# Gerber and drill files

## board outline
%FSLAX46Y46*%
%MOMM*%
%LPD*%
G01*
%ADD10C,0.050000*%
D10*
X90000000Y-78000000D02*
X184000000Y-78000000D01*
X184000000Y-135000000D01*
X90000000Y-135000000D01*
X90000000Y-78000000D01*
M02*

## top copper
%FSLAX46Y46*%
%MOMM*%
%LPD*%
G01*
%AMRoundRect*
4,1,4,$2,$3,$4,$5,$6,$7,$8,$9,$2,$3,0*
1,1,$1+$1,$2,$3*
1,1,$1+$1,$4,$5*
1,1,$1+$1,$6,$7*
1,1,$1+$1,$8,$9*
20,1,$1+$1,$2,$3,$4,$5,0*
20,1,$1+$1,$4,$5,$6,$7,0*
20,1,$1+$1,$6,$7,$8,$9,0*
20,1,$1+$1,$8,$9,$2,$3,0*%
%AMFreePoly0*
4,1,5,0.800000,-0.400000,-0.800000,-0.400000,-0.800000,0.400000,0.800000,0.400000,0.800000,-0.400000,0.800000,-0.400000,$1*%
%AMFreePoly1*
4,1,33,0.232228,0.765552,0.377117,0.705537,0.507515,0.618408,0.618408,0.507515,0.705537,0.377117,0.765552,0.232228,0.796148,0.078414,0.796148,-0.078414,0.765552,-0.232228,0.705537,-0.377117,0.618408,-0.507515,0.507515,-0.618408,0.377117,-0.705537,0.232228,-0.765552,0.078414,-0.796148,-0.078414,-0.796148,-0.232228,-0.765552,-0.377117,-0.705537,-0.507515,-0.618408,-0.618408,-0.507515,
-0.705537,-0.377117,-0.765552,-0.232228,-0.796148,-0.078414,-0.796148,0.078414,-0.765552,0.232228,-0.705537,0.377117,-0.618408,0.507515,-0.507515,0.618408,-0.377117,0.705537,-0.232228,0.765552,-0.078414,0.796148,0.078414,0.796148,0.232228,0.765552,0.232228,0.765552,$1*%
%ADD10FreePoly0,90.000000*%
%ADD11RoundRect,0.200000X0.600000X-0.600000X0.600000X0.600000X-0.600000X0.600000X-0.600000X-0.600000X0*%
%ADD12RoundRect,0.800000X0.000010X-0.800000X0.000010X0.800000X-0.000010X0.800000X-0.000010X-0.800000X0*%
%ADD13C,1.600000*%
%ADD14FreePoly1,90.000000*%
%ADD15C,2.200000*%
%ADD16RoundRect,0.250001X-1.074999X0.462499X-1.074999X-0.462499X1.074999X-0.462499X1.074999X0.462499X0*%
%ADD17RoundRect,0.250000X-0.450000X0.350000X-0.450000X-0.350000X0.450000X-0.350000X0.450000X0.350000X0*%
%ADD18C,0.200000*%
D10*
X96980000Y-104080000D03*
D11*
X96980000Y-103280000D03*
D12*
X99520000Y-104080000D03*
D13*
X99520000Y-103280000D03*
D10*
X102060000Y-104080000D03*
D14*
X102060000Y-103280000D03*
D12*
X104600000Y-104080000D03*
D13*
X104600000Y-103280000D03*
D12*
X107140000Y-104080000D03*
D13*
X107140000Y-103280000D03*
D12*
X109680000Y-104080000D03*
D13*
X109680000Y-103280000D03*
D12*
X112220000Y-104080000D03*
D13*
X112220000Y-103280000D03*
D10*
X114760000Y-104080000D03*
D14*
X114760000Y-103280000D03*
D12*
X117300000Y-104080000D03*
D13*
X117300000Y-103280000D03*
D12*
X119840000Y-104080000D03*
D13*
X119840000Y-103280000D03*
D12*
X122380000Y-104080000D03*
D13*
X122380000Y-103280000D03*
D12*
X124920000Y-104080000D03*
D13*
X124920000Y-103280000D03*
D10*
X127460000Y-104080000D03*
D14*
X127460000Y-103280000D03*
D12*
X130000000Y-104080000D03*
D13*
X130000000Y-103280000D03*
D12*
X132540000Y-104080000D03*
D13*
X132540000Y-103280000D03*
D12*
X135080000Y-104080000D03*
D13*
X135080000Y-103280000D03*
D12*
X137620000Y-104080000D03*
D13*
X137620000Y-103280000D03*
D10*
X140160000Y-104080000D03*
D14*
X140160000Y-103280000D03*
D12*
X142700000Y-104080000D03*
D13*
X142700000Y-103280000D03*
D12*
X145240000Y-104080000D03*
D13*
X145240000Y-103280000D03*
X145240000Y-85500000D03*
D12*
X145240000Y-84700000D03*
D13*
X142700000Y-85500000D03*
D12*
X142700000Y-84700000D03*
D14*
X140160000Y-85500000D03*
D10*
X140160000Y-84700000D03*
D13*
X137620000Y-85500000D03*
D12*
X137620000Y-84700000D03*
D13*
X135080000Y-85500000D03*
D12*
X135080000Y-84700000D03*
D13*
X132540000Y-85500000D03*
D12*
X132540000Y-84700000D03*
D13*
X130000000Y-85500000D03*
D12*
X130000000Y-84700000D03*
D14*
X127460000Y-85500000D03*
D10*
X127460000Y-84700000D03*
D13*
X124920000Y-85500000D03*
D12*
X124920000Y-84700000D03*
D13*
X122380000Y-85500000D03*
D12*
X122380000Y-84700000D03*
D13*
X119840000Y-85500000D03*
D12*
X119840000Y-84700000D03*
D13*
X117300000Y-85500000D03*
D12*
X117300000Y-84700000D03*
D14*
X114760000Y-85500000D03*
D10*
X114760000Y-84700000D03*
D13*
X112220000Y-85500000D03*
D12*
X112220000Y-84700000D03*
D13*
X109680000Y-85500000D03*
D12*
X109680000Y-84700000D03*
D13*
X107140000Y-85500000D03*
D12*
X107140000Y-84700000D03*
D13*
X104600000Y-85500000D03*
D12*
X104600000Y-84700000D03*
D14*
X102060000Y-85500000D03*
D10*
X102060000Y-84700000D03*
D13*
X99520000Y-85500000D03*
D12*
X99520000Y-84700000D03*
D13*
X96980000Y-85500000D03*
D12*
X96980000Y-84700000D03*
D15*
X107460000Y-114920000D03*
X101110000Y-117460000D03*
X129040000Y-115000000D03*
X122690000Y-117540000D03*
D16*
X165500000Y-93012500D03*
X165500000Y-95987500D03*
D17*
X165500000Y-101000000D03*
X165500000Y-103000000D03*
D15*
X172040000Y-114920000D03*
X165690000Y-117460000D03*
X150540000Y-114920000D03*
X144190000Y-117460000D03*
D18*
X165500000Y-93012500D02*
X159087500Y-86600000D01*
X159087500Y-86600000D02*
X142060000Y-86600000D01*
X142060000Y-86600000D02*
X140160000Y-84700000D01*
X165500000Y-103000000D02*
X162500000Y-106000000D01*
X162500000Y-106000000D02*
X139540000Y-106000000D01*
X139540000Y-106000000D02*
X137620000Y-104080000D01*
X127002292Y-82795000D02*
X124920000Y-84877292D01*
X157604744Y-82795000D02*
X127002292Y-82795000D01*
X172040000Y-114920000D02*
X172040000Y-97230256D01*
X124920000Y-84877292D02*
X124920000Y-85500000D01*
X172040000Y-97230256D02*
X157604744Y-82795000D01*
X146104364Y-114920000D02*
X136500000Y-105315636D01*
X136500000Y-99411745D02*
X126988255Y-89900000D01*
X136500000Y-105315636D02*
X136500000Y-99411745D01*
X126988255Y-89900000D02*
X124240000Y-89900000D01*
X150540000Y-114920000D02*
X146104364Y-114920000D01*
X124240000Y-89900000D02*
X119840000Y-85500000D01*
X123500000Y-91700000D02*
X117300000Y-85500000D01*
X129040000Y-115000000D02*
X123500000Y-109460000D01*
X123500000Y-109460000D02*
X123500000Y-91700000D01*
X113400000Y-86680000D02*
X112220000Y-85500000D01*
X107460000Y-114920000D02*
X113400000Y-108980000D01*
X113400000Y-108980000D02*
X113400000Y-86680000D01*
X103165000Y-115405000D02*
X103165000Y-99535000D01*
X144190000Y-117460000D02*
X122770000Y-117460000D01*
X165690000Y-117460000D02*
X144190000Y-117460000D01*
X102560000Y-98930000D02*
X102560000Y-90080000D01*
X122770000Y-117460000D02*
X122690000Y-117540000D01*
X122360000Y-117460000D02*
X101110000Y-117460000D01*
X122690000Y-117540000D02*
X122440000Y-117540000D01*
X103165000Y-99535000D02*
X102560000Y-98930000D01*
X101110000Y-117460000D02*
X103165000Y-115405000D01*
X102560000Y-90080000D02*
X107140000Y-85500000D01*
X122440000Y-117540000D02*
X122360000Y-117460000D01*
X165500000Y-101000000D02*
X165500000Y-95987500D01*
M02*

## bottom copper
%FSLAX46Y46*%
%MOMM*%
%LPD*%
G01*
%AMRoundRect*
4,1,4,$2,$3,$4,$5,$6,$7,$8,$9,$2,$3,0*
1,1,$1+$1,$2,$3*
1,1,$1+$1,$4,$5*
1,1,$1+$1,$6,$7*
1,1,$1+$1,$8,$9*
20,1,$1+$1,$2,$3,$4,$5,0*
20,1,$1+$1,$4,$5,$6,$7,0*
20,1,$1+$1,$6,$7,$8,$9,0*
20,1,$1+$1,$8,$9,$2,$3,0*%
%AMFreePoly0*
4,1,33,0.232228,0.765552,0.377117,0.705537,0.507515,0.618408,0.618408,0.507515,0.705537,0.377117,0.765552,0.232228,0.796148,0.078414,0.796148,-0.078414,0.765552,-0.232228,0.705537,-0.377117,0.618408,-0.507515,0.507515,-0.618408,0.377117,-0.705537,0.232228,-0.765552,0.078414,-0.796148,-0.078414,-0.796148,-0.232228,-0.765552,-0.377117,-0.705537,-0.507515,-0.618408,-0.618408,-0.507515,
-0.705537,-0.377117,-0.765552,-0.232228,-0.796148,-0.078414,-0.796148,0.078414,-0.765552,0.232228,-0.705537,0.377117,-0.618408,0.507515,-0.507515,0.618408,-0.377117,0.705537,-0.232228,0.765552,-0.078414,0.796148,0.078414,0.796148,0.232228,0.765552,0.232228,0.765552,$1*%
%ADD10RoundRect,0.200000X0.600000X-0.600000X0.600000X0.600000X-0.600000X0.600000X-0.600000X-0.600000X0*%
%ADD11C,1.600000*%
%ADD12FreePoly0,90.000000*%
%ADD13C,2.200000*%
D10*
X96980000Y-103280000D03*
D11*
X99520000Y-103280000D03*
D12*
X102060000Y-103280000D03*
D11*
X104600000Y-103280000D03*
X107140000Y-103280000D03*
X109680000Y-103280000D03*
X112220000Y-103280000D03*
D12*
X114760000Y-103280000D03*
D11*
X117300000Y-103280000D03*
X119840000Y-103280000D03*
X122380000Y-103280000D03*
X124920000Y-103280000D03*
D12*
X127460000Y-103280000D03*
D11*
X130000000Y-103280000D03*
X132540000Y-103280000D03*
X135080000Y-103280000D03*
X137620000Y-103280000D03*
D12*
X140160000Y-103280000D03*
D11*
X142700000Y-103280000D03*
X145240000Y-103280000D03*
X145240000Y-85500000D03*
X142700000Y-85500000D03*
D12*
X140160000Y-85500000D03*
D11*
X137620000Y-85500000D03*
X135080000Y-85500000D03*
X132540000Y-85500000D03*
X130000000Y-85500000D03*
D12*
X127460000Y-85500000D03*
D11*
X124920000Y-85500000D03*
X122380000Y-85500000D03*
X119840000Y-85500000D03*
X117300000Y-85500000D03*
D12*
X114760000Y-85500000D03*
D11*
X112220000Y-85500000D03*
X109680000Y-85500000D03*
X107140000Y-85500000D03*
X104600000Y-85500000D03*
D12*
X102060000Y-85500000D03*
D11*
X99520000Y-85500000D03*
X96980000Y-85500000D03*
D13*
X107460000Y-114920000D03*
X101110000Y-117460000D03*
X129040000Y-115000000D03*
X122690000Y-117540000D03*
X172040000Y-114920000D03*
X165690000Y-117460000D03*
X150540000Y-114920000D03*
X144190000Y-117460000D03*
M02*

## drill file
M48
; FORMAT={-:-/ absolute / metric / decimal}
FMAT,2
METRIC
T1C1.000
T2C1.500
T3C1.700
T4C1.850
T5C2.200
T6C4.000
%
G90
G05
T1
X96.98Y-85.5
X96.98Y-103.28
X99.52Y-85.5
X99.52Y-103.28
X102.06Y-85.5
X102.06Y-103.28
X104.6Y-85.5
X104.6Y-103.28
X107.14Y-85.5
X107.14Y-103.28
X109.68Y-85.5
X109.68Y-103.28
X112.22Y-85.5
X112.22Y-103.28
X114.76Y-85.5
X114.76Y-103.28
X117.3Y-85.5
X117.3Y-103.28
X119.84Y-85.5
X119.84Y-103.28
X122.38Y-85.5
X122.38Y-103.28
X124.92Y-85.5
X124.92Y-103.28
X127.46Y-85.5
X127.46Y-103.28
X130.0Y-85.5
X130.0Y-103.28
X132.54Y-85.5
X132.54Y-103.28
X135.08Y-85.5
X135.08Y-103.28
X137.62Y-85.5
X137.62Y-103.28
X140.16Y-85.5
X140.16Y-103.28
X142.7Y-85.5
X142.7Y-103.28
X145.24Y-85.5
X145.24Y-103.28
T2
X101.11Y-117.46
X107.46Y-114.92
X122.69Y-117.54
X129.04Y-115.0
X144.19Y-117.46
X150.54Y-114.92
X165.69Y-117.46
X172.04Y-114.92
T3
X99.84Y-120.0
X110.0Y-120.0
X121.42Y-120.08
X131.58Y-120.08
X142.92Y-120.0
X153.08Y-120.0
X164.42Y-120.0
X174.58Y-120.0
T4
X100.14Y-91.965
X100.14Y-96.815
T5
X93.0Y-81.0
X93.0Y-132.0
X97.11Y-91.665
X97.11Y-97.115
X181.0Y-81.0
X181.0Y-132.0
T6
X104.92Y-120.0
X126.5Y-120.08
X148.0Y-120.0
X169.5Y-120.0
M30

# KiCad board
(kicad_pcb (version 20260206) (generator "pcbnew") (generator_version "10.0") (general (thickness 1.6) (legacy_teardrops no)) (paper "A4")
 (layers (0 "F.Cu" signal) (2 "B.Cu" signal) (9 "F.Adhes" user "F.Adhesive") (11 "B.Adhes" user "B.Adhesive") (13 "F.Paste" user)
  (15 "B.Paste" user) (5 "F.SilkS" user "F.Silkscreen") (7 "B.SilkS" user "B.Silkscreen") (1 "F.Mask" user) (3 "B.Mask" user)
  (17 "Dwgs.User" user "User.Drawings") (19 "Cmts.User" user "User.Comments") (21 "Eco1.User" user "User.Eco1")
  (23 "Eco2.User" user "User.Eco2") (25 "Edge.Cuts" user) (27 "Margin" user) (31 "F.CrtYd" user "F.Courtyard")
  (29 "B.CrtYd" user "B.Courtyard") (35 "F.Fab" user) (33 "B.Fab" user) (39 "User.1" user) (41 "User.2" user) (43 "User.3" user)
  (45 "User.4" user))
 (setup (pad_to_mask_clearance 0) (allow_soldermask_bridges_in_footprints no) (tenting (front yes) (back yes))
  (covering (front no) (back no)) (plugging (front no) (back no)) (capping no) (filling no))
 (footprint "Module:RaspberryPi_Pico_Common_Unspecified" (layer "F.Cu") (at 121.11 94.39 90)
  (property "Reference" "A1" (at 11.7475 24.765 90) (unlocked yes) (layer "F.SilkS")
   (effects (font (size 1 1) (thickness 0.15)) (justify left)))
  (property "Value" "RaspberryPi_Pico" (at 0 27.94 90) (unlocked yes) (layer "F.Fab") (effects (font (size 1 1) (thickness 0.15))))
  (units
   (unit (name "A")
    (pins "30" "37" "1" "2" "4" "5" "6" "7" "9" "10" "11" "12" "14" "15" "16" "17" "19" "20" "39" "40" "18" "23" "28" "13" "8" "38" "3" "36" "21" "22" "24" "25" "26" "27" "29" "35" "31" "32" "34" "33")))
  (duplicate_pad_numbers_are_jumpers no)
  (pad "" np_thru_hole circle (at -2.725 -24 90) (size 2.2 2.2) (drill 2.2) (layers "*.Mask"))
  (pad "" np_thru_hole circle (at -2.425 -20.97 90) (size 1.85 1.85) (drill 1.85) (layers "*.Mask"))
  (pad "" np_thru_hole circle (at 2.425 -20.97 90) (size 1.85 1.85) (drill 1.85) (layers "*.Mask"))
  (pad "" np_thru_hole circle (at 2.725 -24 90) (size 2.2 2.2) (drill 2.2) (layers "*.Mask"))
  (pad "1" smd custom (at -9.69 -24.13 90) (size 1.6 0.8) (layers "F.Cu" "F.Mask") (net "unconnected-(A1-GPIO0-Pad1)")
   (options (clearance outline) (anchor rect)) (primitives))
  (pad "1" thru_hole roundrect (at -8.89 -24.13 90) (size 1.6 1.6) (drill 1) (layers "*.Cu" "*.Mask") (remove_unused_layers no)
   (roundrect_rratio 0.125) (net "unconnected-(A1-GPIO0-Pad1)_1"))
  (pad "2" smd roundrect (at -9.69 -21.59 90) (size 3.2 1.6) (layers "F.Cu" "F.Mask") (roundrect_rratio 0.5)
   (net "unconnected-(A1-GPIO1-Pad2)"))
  (pad "2" thru_hole circle (at -8.89 -21.59 90) (size 1.6 1.6) (drill 1) (layers "*.Cu" "*.Mask") (remove_unused_layers no)
   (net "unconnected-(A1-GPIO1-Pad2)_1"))
  (pad "3" smd custom (at -9.69 -19.05 90) (size 1.6 0.8) (layers "F.Cu" "F.Mask") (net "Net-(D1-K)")
   (options (clearance outline) (anchor rect)) (primitives))
  (pad "3" thru_hole custom (at -8.89 -19.05 90) (size 1.6 1.6) (drill 1) (layers "*.Cu" "*.Mask") (remove_unused_layers no)
   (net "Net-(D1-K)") (options (clearance outline) (anchor circle)) (primitives))
  (pad "4" smd roundrect (at -9.69 -16.51 90) (size 3.2 1.6) (layers "F.Cu" "F.Mask") (roundrect_rratio 0.5)
   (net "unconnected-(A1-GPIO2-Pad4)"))
  (pad "4" thru_hole circle (at -8.89 -16.51 90) (size 1.6 1.6) (drill 1) (layers "*.Cu" "*.Mask") (remove_unused_layers no)
   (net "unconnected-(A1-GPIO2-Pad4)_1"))
  (pad "5" smd roundrect (at -9.69 -13.97 90) (size 3.2 1.6) (layers "F.Cu" "F.Mask") (roundrect_rratio 0.5)
   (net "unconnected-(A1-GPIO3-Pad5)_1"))
  (pad "5" thru_hole circle (at -8.89 -13.97 90) (size 1.6 1.6) (drill 1) (layers "*.Cu" "*.Mask") (remove_unused_layers no)
   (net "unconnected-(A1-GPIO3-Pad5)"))
  (pad "6" smd roundrect (at -9.69 -11.43 90) (size 3.2 1.6) (layers "F.Cu" "F.Mask") (roundrect_rratio 0.5)
   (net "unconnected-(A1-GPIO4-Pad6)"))
  (pad "6" thru_hole circle (at -8.89 -11.43 90) (size 1.6 1.6) (drill 1) (layers "*.Cu" "*.Mask") (remove_unused_layers no)
   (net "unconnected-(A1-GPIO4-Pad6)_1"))
  (pad "7" smd roundrect (at -9.69 -8.89 90) (size 3.2 1.6) (layers "F.Cu" "F.Mask") (roundrect_rratio 0.5)
   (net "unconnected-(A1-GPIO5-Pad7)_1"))
  (pad "7" thru_hole circle (at -8.89 -8.89 90) (size 1.6 1.6) (drill 1) (layers "*.Cu" "*.Mask") (remove_unused_layers no)
   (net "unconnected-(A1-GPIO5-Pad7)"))
  (pad "8" smd custom (at -9.69 -6.35 90) (size 1.6 0.8) (layers "F.Cu" "F.Mask") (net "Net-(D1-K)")
   (options (clearance outline) (anchor rect)) (primitives))
  (pad "8" thru_hole custom (at -8.89 -6.35 90) (size 1.6 1.6) (drill 1) (layers "*.Cu" "*.Mask") (remove_unused_layers no)
   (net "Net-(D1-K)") (options (clearance outline) (anchor circle)) (primitives))
  (pad "9" smd roundrect (at -9.69 -3.81 90) (size 3.2 1.6) (layers "F.Cu" "F.Mask") (roundrect_rratio 0.5)
   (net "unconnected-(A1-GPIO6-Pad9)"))
  (pad "9" thru_hole circle (at -8.89 -3.81 90) (size 1.6 1.6) (drill 1) (layers "*.Cu" "*.Mask") (remove_unused_layers no)
   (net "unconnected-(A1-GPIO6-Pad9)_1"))
  (pad "10" smd roundrect (at -9.69 -1.27 90) (size 3.2 1.6) (layers "F.Cu" "F.Mask") (roundrect_rratio 0.5)
   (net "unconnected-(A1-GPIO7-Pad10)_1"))
  (pad "10" thru_hole circle (at -8.89 -1.27 90) (size 1.6 1.6) (drill 1) (layers "*.Cu" "*.Mask") (remove_unused_layers no)
   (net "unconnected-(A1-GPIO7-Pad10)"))
  (pad "11" smd roundrect (at -9.69 1.27 90) (size 3.2 1.6) (layers "F.Cu" "F.Mask") (roundrect_rratio 0.5)
   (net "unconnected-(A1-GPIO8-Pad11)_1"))
  (pad "11" thru_hole circle (at -8.89 1.27 90) (size 1.6 1.6) (drill 1) (layers "*.Cu" "*.Mask") (remove_unused_layers no)
   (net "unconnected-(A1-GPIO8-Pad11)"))
  (pad "12" smd roundrect (at -9.69 3.81 90) (size 3.2 1.6) (layers "F.Cu" "F.Mask") (roundrect_rratio 0.5)
   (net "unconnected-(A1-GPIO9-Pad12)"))
  (pad "12" thru_hole circle (at -8.89 3.81 90) (size 1.6 1.6) (drill 1) (layers "*.Cu" "*.Mask") (remove_unused_layers no)
   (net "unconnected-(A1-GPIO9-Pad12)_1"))
  (pad "13" smd custom (at -9.69 6.35 90) (size 1.6 0.8) (layers "F.Cu" "F.Mask") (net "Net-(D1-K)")
   (options (clearance outline) (anchor rect)) (primitives))
  (pad "13" thru_hole custom (at -8.89 6.35 90) (size 1.6 1.6) (drill 1) (layers "*.Cu" "*.Mask") (remove_unused_layers no)
   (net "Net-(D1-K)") (options (clearance outline) (anchor circle)) (primitives))
  (pad "14" smd roundrect (at -9.69 8.89 90) (size 3.2 1.6) (layers "F.Cu" "F.Mask") (roundrect_rratio 0.5)
   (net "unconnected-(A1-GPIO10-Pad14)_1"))
  (pad "14" thru_hole circle (at -8.89 8.89 90) (size 1.6 1.6) (drill 1) (layers "*.Cu" "*.Mask") (remove_unused_layers no)
   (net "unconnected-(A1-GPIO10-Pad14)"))
  (pad "15" smd roundrect (at -9.69 11.43 90) (size 3.2 1.6) (layers "F.Cu" "F.Mask") (roundrect_rratio 0.5)
   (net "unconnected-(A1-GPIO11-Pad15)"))
  (pad "15" thru_hole circle (at -8.89 11.43 90) (size 1.6 1.6) (drill 1) (layers "*.Cu" "*.Mask") (remove_unused_layers no)
   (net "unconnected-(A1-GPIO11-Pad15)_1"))
  (pad "16" smd roundrect (at -9.69 13.97 90) (size 3.2 1.6) (layers "F.Cu" "F.Mask") (roundrect_rratio 0.5)
   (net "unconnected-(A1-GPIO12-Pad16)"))
  (pad "16" thru_hole circle (at -8.89 13.97 90) (size 1.6 1.6) (drill 1) (layers "*.Cu" "*.Mask") (remove_unused_layers no)
   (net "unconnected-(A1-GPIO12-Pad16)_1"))
  (pad "17" smd roundrect (at -9.69 16.51 90) (size 3.2 1.6) (layers "F.Cu" "F.Mask") (roundrect_rratio 0.5) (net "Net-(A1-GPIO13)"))
  (pad "17" thru_hole circle (at -8.89 16.51 90) (size 1.6 1.6) (drill 1) (layers "*.Cu" "*.Mask") (remove_unused_layers no)
   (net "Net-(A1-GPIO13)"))
  (pad "18" smd custom (at -9.69 19.05 90) (size 1.6 0.8) (layers "F.Cu" "F.Mask") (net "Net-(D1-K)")
   (options (clearance outline) (anchor rect)) (primitives))
  (pad "18" thru_hole custom (at -8.89 19.05 90) (size 1.6 1.6) (drill 1) (layers "*.Cu" "*.Mask") (remove_unused_layers no)
   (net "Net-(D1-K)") (options (clearance outline) (anchor circle)) (primitives))
  (pad "19" smd roundrect (at -9.69 21.59 90) (size 3.2 1.6) (layers "F.Cu" "F.Mask") (roundrect_rratio 0.5)
   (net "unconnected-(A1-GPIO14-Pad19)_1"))
  (pad "19" thru_hole circle (at -8.89 21.59 90) (size 1.6 1.6) (drill 1) (layers "*.Cu" "*.Mask") (remove_unused_layers no)
   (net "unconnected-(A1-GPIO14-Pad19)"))
  (pad "20" smd roundrect (at -9.69 24.13 90) (size 3.2 1.6) (layers "F.Cu" "F.Mask") (roundrect_rratio 0.5)
   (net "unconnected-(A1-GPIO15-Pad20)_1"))
  (pad "20" thru_hole circle (at -8.89 24.13 90) (size 1.6 1.6) (drill 1) (layers "*.Cu" "*.Mask") (remove_unused_layers no)
   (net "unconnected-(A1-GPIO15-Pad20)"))
  (pad "21" thru_hole circle (at 8.89 24.13 90) (size 1.6 1.6) (drill 1) (layers "*.Cu" "*.Mask") (remove_unused_layers no)
   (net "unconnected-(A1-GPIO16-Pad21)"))
  (pad "21" smd roundrect (at 9.69 24.13 90) (size 3.2 1.6) (layers "F.Cu" "F.Mask") (roundrect_rratio 0.5)
   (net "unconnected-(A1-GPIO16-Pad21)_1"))
  (pad "22" thru_hole circle (at 8.89 21.59 90) (size 1.6 1.6) (drill 1) (layers "*.Cu" "*.Mask") (remove_unused_layers no)
   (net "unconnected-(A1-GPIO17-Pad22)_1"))
  (pad "22" smd roundrect (at 9.69 21.59 90) (size 3.2 1.6) (layers "F.Cu" "F.Mask") (roundrect_rratio 0.5)
   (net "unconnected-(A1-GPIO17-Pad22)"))
  (pad "23" thru_hole custom (at 8.89 19.05 90) (size 1.6 1.6) (drill 1) (layers "*.Cu" "*.Mask") (remove_unused_layers no)
   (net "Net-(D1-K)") (options (clearance outline) (anchor circle)) (primitives))
  (pad "23" smd custom (at 9.69 19.05 90) (size 1.6 0.8) (layers "F.Cu" "F.Mask") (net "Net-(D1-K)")
   (options (clearance outline) (anchor rect)) (primitives))
  (pad "24" thru_hole circle (at 8.89 16.51 90) (size 1.6 1.6) (drill 1) (layers "*.Cu" "*.Mask") (remove_unused_layers no)
   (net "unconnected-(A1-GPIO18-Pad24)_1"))
  (pad "24" smd roundrect (at 9.69 16.51 90) (size 3.2 1.6) (layers "F.Cu" "F.Mask") (roundrect_rratio 0.5)
   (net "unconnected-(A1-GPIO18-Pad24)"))
  (pad "25" thru_hole circle (at 8.89 13.97 90) (size 1.6 1.6) (drill 1) (layers "*.Cu" "*.Mask") (remove_unused_layers no)
   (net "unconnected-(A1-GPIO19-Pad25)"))
  (pad "25" smd roundrect (at 9.69 13.97 90) (size 3.2 1.6) (layers "F.Cu" "F.Mask") (roundrect_rratio 0.5)
   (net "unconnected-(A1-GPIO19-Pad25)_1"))
  (pad "26" thru_hole circle (at 8.89 11.43 90) (size 1.6 1.6) (drill 1) (layers "*.Cu" "*.Mask") (remove_unused_layers no)
   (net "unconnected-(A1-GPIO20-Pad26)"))
  (pad "26" smd roundrect (at 9.69 11.43 90) (size 3.2 1.6) (layers "F.Cu" "F.Mask") (roundrect_rratio 0.5)
   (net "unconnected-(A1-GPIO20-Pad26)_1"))
  (pad "27" thru_hole circle (at 8.89 8.89 90) (size 1.6 1.6) (drill 1) (layers "*.Cu" "*.Mask") (remove_unused_layers no)
   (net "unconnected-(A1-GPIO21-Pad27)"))
  (pad "27" smd roundrect (at 9.69 8.89 90) (size 3.2 1.6) (layers "F.Cu" "F.Mask") (roundrect_rratio 0.5)
   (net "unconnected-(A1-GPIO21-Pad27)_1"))
  (pad "28" thru_hole custom (at 8.89 6.35 90) (size 1.6 1.6) (drill 1) (layers "*.Cu" "*.Mask") (remove_unused_layers no)
   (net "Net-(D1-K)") (options (clearance outline) (anchor circle)) (primitives))
  (pad "28" smd custom (at 9.69 6.35 90) (size 1.6 0.8) (layers "F.Cu" "F.Mask") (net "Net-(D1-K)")
   (options (clearance outline) (anchor rect)) (primitives))
  (pad "29" thru_hole circle (at 8.89 3.81 90) (size 1.6 1.6) (drill 1) (layers "*.Cu" "*.Mask") (remove_unused_layers no)
   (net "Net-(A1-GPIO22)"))
  (pad "29" smd roundrect (at 9.69 3.81 90) (size 3.2 1.6) (layers "F.Cu" "F.Mask") (roundrect_rratio 0.5) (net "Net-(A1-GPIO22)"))
  (pad "30" thru_hole circle (at 8.89 1.27 90) (size 1.6 1.6) (drill 1) (layers "*.Cu" "*.Mask") (remove_unused_layers no)
   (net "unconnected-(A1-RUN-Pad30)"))
  (pad "30" smd roundrect (at 9.69 1.27 90) (size 3.2 1.6) (layers "F.Cu" "F.Mask") (roundrect_rratio 0.5)
   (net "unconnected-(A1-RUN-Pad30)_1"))
  (pad "31" thru_hole circle (at 8.89 -1.27 90) (size 1.6 1.6) (drill 1) (layers "*.Cu" "*.Mask") (remove_unused_layers no)
   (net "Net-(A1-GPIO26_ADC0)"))
  (pad "31" smd roundrect (at 9.69 -1.27 90) (size 3.2 1.6) (layers "F.Cu" "F.Mask") (roundrect_rratio 0.5) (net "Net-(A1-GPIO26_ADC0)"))
  (pad "32" thru_hole circle (at 8.89 -3.81 90) (size 1.6 1.6) (drill 1) (layers "*.Cu" "*.Mask") (remove_unused_layers no)
   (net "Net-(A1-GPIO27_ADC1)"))
  (pad "32" smd roundrect (at 9.69 -3.81 90) (size 3.2 1.6) (layers "F.Cu" "F.Mask") (roundrect_rratio 0.5) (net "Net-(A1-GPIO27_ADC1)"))
  (pad "33" thru_hole custom (at 8.89 -6.35 90) (size 1.6 1.6) (drill 1) (layers "*.Cu" "*.Mask") (remove_unused_layers no)
   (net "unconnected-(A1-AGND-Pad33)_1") (options (clearance outline) (anchor circle)) (primitives))
  (pad "33" smd custom (at 9.69 -6.35 90) (size 1.6 0.8) (layers "F.Cu" "F.Mask") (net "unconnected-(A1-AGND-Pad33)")
   (options (clearance outline) (anchor rect)) (primitives))
  (pad "34" thru_hole circle (at 8.89 -8.89 90) (size 1.6 1.6) (drill 1) (layers "*.Cu" "*.Mask") (remove_unused_layers no)
   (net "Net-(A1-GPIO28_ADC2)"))
  (pad "34" smd roundrect (at 9.69 -8.89 90) (size 3.2 1.6) (layers "F.Cu" "F.Mask") (roundrect_rratio 0.5) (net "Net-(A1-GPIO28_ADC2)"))
  (pad "35" thru_hole circle (at 8.89 -11.43 90) (size 1.6 1.6) (drill 1) (layers "*.Cu" "*.Mask") (remove_unused_layers no)
   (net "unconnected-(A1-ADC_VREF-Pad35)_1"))
  (pad "35" smd roundrect (at 9.69 -11.43 90) (size 3.2 1.6) (layers "F.Cu" "F.Mask") (roundrect_rratio 0.5)
   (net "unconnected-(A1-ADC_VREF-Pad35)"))
  (pad "36" thru_hole circle (at 8.89 -13.97 90) (size 1.6 1.6) (drill 1) (layers "*.Cu" "*.Mask") (remove_unused_layers no)
   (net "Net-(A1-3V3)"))
  (pad "36" smd roundrect (at 9.69 -13.97 90) (size 3.2 1.6) (layers "F.Cu" "F.Mask") (roundrect_rratio 0.5) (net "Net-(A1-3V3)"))
  (pad "37" thru_hole circle (at 8.89 -16.51 90) (size 1.6 1.6) (drill 1) (layers "*.Cu" "*.Mask") (remove_unused_layers no)
   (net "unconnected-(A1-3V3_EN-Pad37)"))
  (pad "37" smd roundrect (at 9.69 -16.51 90) (size 3.2 1.6) (layers "F.Cu" "F.Mask") (roundrect_rratio 0.5)
   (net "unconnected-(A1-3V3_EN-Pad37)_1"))
  (pad "38" thru_hole custom (at 8.89 -19.05 90) (size 1.6 1.6) (drill 1) (layers "*.Cu" "*.Mask") (remove_unused_layers no)
   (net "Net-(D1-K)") (options (clearance outline) (anchor circle)) (primitives))
  (pad "38" smd custom (at 9.69 -19.05 90) (size 1.6 0.8) (layers "F.Cu" "F.Mask") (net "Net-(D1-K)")
   (options (clearance outline) (anchor rect)) (primitives))
  (pad "39" thru_hole circle (at 8.89 -21.59 90) (size 1.6 1.6) (drill 1) (layers "*.Cu" "*.Mask") (remove_unused_layers no)
   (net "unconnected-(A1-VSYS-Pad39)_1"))
  (pad "39" smd roundrect (at 9.69 -21.59 90) (size 3.2 1.6) (layers "F.Cu" "F.Mask") (roundrect_rratio 0.5)
   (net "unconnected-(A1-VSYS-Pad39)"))
  (pad "40" thru_hole circle (at 8.89 -24.13 90) (size 1.6 1.6) (drill 1) (layers "*.Cu" "*.Mask") (remove_unused_layers no)
   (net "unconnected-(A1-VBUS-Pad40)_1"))
  (pad "40" smd roundrect (at 9.69 -24.13 90) (size 3.2 1.6) (layers "F.Cu" "F.Mask") (roundrect_rratio 0.5)
   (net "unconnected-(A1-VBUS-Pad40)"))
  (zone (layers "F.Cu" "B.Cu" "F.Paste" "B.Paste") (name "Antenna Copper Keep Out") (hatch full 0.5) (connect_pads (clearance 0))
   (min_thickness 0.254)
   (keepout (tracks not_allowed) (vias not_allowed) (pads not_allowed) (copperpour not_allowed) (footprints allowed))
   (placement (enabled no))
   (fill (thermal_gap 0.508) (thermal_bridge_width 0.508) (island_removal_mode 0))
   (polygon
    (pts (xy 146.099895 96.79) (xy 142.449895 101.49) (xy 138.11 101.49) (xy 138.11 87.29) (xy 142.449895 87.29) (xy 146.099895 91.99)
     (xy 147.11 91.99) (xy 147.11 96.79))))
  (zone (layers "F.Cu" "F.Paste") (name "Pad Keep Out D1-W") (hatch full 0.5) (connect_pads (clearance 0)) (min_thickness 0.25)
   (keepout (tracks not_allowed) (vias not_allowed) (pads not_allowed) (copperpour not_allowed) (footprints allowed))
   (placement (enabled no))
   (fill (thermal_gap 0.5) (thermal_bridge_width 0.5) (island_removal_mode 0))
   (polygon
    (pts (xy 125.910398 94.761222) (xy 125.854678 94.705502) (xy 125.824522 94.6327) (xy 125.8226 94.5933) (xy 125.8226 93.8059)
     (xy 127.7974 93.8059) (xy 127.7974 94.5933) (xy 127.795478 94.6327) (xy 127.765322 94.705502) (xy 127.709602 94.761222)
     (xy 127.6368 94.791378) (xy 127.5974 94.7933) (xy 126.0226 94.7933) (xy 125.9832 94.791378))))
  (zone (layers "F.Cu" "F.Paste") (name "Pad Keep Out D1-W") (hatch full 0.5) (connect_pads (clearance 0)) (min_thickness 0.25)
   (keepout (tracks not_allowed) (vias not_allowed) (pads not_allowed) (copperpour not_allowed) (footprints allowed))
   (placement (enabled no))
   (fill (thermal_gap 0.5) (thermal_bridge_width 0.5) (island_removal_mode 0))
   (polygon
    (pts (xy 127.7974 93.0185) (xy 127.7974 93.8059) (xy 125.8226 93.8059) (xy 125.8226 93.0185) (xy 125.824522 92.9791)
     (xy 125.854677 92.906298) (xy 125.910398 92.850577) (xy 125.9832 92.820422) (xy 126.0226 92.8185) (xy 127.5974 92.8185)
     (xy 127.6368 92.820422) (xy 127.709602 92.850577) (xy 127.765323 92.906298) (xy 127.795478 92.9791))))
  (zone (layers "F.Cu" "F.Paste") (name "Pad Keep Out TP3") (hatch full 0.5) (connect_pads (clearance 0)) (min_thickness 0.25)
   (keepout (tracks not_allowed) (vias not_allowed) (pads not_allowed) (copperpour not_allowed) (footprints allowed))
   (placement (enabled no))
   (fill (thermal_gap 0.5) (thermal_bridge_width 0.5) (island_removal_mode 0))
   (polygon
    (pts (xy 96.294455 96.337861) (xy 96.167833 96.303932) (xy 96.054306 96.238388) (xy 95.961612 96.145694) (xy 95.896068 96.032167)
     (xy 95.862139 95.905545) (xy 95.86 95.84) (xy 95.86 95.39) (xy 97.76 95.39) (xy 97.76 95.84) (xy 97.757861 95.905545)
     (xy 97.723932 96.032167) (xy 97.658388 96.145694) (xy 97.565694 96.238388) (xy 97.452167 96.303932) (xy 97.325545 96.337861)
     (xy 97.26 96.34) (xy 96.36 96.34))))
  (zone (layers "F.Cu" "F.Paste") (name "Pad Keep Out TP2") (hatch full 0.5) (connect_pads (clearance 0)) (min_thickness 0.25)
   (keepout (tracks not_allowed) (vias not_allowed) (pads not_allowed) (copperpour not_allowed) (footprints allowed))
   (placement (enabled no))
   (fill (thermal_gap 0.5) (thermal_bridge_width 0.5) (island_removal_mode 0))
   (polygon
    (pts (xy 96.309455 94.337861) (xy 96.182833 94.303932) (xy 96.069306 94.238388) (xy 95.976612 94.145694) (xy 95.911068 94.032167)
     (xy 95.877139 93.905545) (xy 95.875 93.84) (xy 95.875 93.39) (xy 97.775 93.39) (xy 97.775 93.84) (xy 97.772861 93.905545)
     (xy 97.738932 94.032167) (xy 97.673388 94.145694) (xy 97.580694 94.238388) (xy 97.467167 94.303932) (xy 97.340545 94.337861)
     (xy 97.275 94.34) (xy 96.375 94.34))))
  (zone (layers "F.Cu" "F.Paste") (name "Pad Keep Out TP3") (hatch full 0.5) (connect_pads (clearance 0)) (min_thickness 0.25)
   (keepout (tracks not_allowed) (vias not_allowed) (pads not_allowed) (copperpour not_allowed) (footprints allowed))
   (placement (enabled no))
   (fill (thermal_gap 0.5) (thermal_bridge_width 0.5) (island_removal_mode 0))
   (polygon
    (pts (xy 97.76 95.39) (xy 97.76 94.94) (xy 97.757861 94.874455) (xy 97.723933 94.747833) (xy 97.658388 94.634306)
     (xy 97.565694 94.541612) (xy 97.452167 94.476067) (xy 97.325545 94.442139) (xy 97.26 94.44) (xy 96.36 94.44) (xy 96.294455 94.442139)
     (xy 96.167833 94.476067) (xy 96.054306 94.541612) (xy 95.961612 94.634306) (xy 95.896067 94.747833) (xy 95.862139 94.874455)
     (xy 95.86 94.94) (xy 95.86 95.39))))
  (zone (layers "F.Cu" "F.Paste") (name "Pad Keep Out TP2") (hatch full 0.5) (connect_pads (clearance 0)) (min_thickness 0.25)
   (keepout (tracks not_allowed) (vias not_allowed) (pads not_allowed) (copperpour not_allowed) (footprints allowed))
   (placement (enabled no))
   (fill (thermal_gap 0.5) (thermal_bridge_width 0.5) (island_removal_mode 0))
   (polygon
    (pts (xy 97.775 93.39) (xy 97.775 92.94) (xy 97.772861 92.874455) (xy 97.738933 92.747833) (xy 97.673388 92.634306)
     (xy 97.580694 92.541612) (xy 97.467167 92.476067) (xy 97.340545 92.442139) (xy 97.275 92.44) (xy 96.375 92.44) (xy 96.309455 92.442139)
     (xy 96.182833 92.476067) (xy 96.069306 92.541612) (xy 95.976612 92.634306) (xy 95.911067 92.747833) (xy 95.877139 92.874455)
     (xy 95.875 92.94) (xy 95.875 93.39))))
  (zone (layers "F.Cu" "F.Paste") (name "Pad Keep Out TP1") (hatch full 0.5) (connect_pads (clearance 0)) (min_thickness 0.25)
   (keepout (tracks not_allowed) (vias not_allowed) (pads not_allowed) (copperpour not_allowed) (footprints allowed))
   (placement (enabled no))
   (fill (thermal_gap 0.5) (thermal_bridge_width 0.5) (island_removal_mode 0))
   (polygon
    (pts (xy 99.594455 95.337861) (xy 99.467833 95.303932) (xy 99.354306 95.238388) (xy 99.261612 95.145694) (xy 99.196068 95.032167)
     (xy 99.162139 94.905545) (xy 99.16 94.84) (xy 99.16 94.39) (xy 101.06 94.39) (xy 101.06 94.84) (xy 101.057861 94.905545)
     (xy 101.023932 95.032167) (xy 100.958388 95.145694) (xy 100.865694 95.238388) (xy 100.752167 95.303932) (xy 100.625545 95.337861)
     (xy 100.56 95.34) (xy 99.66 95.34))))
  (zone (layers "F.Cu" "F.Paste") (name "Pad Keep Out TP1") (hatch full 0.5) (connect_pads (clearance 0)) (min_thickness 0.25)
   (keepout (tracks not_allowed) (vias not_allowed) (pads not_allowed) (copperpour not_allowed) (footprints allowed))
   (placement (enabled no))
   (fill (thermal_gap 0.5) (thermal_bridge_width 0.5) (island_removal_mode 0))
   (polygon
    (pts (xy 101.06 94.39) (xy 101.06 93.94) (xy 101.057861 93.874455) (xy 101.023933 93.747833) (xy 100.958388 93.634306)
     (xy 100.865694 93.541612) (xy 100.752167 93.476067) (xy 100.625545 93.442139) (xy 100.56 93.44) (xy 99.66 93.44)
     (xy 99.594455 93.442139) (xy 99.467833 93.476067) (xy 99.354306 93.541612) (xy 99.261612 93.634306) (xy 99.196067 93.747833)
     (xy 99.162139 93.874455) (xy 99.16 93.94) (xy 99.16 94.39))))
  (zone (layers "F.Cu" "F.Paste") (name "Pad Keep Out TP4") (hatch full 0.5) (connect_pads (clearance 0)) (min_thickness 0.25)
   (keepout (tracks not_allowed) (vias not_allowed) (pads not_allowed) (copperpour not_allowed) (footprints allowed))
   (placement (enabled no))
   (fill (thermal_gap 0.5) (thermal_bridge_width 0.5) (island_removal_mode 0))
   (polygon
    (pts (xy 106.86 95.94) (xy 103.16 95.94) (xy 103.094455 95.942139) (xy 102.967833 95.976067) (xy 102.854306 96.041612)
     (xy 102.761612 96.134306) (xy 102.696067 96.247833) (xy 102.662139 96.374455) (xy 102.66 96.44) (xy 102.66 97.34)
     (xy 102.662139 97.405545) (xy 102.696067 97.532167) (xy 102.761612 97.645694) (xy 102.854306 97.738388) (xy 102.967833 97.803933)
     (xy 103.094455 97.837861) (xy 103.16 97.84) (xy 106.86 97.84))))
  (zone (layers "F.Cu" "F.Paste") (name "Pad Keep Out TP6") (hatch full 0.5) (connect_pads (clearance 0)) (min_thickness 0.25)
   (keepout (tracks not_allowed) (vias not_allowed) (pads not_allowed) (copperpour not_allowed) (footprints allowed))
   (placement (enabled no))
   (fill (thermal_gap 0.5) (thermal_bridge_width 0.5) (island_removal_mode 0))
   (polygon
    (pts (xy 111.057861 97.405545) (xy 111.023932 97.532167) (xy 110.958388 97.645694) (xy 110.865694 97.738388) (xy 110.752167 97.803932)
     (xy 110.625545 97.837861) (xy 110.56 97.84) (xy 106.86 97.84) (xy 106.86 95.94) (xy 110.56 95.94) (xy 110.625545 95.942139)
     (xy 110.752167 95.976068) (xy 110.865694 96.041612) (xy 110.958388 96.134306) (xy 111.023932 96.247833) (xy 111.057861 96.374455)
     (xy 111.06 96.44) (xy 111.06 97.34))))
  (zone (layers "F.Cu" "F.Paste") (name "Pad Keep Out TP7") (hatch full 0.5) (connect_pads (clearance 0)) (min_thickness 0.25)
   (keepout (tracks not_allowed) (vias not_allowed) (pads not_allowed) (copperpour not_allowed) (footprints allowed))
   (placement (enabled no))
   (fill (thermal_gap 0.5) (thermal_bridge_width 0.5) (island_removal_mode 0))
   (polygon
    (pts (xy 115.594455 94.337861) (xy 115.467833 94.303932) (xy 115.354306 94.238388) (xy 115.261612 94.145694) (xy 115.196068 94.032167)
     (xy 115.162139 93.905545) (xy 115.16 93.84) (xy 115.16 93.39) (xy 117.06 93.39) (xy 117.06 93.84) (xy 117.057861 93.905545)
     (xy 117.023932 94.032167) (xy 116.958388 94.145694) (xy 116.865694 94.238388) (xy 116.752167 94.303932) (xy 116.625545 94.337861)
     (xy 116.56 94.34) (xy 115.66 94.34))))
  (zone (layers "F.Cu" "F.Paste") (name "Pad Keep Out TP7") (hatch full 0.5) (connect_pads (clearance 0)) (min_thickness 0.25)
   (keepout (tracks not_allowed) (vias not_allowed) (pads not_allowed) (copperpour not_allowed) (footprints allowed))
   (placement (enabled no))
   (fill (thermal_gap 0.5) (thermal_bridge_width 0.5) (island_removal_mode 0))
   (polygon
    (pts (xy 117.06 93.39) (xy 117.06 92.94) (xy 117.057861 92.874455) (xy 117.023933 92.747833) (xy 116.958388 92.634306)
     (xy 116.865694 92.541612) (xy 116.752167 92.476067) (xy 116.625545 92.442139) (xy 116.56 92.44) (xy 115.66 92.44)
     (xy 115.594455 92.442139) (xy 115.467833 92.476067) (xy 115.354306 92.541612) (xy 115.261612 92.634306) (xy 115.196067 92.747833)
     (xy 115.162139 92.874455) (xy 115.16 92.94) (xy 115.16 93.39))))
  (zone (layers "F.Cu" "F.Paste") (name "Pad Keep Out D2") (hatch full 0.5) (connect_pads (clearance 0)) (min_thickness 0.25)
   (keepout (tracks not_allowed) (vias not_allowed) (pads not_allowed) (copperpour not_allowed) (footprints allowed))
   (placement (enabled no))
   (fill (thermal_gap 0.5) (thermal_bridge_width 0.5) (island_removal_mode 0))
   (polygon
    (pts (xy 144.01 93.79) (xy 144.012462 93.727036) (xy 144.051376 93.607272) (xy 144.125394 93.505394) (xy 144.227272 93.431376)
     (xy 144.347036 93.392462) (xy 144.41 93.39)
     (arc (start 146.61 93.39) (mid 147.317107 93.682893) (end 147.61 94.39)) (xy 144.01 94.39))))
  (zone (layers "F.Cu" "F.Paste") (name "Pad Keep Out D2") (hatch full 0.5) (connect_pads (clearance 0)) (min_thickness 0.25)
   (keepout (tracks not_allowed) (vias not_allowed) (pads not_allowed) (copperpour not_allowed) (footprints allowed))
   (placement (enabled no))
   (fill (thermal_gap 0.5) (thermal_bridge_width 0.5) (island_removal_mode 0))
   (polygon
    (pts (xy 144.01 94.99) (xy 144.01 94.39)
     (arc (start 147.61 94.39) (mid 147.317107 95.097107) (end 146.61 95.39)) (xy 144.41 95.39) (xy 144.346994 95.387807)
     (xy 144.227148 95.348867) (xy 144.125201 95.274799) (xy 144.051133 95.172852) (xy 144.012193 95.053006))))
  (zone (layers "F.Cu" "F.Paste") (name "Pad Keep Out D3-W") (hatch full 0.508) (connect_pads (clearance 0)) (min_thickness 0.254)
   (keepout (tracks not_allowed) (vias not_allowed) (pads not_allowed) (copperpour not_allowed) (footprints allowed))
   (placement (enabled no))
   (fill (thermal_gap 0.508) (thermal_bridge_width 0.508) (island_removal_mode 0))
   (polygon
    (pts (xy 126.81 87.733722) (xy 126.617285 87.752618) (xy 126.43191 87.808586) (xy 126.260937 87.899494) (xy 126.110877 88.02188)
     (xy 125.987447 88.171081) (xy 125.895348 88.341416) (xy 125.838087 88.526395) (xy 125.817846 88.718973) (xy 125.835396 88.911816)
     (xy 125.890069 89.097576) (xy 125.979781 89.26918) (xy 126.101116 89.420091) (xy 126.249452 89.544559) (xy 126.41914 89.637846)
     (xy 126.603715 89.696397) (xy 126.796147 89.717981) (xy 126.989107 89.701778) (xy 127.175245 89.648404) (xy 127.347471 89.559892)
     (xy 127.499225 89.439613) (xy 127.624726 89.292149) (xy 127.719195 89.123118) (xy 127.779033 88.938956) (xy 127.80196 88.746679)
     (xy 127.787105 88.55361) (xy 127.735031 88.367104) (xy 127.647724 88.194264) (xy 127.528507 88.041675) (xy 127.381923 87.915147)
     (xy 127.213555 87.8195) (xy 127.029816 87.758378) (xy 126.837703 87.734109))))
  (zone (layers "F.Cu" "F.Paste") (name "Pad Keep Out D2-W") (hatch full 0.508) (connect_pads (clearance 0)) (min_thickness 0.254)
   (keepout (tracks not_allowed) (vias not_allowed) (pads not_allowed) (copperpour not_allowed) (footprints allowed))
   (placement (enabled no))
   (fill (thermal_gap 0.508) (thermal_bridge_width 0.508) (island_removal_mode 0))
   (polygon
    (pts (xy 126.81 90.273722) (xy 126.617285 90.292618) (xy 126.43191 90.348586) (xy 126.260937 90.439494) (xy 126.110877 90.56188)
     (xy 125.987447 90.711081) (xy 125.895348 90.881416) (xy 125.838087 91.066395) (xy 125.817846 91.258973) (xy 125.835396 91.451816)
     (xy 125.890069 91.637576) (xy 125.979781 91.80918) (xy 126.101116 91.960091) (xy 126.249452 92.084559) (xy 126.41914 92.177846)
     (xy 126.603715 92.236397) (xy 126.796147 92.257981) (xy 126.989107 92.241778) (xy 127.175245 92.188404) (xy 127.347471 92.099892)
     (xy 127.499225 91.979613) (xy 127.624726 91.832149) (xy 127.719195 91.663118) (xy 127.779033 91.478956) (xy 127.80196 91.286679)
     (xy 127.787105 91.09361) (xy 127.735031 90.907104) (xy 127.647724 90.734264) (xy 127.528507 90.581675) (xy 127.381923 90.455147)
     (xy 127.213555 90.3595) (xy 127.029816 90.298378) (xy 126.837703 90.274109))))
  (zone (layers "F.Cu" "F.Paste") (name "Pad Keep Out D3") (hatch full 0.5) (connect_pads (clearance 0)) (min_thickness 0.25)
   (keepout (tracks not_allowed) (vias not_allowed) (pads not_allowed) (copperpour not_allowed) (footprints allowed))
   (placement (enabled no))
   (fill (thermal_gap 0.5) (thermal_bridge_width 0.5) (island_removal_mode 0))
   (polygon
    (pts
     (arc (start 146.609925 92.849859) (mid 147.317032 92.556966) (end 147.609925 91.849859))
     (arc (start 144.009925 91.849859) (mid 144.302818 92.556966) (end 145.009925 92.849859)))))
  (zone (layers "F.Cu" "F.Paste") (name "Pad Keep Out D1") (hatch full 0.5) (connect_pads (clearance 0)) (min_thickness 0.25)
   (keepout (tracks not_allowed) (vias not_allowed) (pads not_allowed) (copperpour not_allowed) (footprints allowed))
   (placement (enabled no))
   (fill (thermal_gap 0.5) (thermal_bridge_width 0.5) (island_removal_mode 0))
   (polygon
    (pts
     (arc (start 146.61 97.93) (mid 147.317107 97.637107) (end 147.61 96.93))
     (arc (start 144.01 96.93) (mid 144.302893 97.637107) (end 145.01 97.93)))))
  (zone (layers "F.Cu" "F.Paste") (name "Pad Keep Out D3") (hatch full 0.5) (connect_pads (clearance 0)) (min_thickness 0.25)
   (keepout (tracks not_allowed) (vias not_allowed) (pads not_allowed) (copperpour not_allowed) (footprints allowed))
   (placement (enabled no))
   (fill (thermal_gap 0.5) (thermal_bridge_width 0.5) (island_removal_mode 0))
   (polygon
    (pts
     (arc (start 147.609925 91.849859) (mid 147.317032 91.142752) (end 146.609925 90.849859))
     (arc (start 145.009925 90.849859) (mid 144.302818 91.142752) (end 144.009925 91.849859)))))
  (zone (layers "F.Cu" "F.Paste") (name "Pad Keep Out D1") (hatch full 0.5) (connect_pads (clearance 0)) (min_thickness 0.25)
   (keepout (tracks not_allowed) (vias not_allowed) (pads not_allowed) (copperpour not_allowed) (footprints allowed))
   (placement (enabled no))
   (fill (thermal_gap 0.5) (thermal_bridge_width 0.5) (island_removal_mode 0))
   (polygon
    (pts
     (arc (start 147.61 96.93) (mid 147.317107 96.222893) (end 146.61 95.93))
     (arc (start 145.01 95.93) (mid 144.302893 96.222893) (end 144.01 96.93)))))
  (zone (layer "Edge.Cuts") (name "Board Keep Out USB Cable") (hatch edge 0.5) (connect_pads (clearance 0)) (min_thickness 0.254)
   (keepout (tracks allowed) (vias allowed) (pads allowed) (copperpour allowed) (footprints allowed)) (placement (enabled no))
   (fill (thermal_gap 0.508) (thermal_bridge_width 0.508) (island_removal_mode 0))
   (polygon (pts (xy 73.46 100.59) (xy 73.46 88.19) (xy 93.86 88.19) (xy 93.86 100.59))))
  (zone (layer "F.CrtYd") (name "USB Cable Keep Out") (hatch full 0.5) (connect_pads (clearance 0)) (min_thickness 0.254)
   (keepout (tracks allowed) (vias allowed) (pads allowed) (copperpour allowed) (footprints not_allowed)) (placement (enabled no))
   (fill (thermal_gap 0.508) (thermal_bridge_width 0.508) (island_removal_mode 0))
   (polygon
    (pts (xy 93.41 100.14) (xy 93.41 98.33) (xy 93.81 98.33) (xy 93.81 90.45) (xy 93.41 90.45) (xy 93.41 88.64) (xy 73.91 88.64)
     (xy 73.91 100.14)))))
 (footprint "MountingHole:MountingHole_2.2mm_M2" (layer "F.Cu") (at 181 81)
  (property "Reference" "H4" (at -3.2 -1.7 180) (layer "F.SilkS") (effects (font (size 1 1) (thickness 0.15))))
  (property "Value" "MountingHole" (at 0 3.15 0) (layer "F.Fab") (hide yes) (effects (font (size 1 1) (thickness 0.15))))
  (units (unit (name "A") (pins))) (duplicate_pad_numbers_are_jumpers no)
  (pad "" np_thru_hole circle (at 0 0) (size 2.2 2.2) (drill 2.2) (layers "*.Cu" "*.Mask")))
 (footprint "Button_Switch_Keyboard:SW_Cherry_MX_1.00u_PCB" (layer "F.Cu") (at 107.46 114.92)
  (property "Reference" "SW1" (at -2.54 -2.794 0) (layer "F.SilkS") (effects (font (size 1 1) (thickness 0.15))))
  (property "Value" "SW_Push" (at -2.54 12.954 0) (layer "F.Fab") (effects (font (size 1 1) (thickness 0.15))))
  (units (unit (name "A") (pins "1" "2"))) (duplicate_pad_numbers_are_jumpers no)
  (pad "" np_thru_hole circle (at -7.62 5.08) (size 1.7 1.7) (drill 1.7) (layers "*.Cu" "*.Mask"))
  (pad "" np_thru_hole circle (at -2.54 5.08) (size 4 4) (drill 4) (layers "*.Cu" "*.Mask"))
  (pad "" np_thru_hole circle (at 2.54 5.08) (size 1.7 1.7) (drill 1.7) (layers "*.Cu" "*.Mask"))
  (pad "1" thru_hole circle (at 0 0) (size 2.2 2.2) (drill 1.5) (layers "*.Cu" "*.Mask") (remove_unused_layers no)
   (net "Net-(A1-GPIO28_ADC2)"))
  (pad "2" thru_hole circle (at -6.35 2.54) (size 2.2 2.2) (drill 1.5) (layers "*.Cu" "*.Mask") (remove_unused_layers no)
   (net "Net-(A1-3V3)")))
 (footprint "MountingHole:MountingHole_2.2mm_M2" (layer "F.Cu") (at 181 132)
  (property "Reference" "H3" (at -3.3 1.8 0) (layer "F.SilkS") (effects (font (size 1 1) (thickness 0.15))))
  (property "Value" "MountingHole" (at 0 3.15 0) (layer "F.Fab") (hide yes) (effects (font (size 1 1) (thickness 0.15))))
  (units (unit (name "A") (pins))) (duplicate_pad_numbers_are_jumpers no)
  (pad "" np_thru_hole circle (at 0 0) (size 2.2 2.2) (drill 2.2) (layers "*.Cu" "*.Mask")))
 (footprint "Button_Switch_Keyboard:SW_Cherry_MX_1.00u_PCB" (layer "F.Cu") (at 129.04 115)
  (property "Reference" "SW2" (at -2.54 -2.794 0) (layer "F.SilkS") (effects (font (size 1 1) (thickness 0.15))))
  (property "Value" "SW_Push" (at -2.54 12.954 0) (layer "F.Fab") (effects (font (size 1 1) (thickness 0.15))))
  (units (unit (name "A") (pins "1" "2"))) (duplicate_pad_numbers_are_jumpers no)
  (pad "" np_thru_hole circle (at -7.62 5.08) (size 1.7 1.7) (drill 1.7) (layers "*.Cu" "*.Mask"))
  (pad "" np_thru_hole circle (at -2.54 5.08) (size 4 4) (drill 4) (layers "*.Cu" "*.Mask"))
  (pad "" np_thru_hole circle (at 2.54 5.08) (size 1.7 1.7) (drill 1.7) (layers "*.Cu" "*.Mask"))
  (pad "1" thru_hole circle (at 0 0) (size 2.2 2.2) (drill 1.5) (layers "*.Cu" "*.Mask") (remove_unused_layers no)
   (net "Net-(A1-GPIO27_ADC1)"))
  (pad "2" thru_hole circle (at -6.35 2.54) (size 2.2 2.2) (drill 1.5) (layers "*.Cu" "*.Mask") (remove_unused_layers no)
   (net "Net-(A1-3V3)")))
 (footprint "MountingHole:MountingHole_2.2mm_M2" (layer "F.Cu") (at 93 81 180)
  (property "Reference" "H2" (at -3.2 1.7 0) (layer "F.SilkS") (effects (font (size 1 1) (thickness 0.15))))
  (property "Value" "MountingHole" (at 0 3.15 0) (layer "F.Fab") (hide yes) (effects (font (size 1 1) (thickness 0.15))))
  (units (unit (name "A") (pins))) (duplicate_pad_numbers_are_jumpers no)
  (pad "" np_thru_hole circle (at 0 0 180) (size 2.2 2.2) (drill 2.2) (layers "*.Cu" "*.Mask")))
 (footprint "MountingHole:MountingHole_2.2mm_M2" (layer "F.Cu") (at 93 132 180)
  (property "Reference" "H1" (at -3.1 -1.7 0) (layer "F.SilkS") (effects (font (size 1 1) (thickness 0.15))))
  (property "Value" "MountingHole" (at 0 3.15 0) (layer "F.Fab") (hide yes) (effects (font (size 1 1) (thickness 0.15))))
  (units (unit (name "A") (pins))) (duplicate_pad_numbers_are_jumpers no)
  (pad "" np_thru_hole circle (at 0 0 180) (size 2.2 2.2) (drill 2.2) (layers "*.Cu" "*.Mask")))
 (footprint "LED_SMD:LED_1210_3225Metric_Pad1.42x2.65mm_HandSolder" (layer "F.Cu") (at 165.5 94.5 -90)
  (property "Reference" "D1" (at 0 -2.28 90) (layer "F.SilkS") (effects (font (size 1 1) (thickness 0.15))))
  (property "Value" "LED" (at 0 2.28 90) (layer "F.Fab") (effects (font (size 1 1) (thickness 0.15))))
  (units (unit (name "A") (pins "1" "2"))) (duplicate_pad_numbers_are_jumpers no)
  (pad "1" smd roundrect (at -1.4875 0 270) (size 1.425 2.65) (layers "F.Cu" "F.Mask" "F.Paste") (roundrect_rratio 0.175439)
   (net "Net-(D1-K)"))
  (pad "2" smd roundrect (at 1.4875 0 270) (size 1.425 2.65) (layers "F.Cu" "F.Mask" "F.Paste") (roundrect_rratio 0.175439)
   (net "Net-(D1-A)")))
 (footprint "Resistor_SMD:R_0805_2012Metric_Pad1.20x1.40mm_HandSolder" (layer "F.Cu") (at 165.5 102 -90)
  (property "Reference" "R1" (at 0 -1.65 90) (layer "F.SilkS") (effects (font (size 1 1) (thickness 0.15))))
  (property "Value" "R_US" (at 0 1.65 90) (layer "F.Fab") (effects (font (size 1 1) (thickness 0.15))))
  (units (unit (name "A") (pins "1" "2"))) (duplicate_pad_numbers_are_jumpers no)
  (pad "1" smd roundrect (at -1 0 270) (size 1.2 1.4) (layers "F.Cu" "F.Mask" "F.Paste") (roundrect_rratio 0.208333) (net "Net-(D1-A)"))
  (pad "2" smd roundrect (at 1 0 270) (size 1.2 1.4) (layers "F.Cu" "F.Mask" "F.Paste") (roundrect_rratio 0.208333) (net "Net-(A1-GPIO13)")))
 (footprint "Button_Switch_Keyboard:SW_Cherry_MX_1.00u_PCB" (layer "F.Cu") (at 172.04 114.92)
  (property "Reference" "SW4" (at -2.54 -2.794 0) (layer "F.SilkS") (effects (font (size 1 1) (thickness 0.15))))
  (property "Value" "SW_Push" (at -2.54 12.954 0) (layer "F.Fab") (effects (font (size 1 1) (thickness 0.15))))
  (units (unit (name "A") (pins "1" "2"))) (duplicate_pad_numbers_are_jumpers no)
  (pad "" np_thru_hole circle (at -7.62 5.08) (size 1.7 1.7) (drill 1.7) (layers "*.Cu" "*.Mask"))
  (pad "" np_thru_hole circle (at -2.54 5.08) (size 4 4) (drill 4) (layers "*.Cu" "*.Mask"))
  (pad "" np_thru_hole circle (at 2.54 5.08) (size 1.7 1.7) (drill 1.7) (layers "*.Cu" "*.Mask"))
  (pad "1" thru_hole circle (at 0 0) (size 2.2 2.2) (drill 1.5) (layers "*.Cu" "*.Mask") (remove_unused_layers no) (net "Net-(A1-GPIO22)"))
  (pad "2" thru_hole circle (at -6.35 2.54) (size 2.2 2.2) (drill 1.5) (layers "*.Cu" "*.Mask") (remove_unused_layers no)
   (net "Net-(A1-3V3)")))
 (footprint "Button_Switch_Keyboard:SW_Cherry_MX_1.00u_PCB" (layer "F.Cu") (at 150.54 114.92)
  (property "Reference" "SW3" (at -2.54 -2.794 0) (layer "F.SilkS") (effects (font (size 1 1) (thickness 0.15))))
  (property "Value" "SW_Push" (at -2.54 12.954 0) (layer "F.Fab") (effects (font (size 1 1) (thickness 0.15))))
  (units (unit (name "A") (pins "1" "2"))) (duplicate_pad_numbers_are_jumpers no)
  (pad "" np_thru_hole circle (at -7.62 5.08) (size 1.7 1.7) (drill 1.7) (layers "*.Cu" "*.Mask"))
  (pad "" np_thru_hole circle (at -2.54 5.08) (size 4 4) (drill 4) (layers "*.Cu" "*.Mask"))
  (pad "" np_thru_hole circle (at 2.54 5.08) (size 1.7 1.7) (drill 1.7) (layers "*.Cu" "*.Mask"))
  (pad "1" thru_hole circle (at 0 0) (size 2.2 2.2) (drill 1.5) (layers "*.Cu" "*.Mask") (remove_unused_layers no)
   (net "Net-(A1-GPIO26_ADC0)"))
  (pad "2" thru_hole circle (at -6.35 2.54) (size 2.2 2.2) (drill 1.5) (layers "*.Cu" "*.Mask") (remove_unused_layers no)
   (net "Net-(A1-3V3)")))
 (gr_rect (start 90 78) (end 184 135) (stroke (width 0.05) (type solid)) (fill no) (layer "Edge.Cuts"))
 (segment (start 165.5 93.0125) (end 159.0875 86.6) (width 0.2) (layer "F.Cu") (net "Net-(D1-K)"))
 (segment (start 159.0875 86.6) (end 142.06 86.6) (width 0.2) (layer "F.Cu") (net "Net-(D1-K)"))
 (segment (start 142.06 86.6) (end 140.16 84.7) (width 0.2) (layer "F.Cu") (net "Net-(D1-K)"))
 (segment (start 165.5 103) (end 162.5 106) (width 0.2) (layer "F.Cu") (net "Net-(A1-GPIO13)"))
 (segment (start 162.5 106) (end 139.54 106) (width 0.2) (layer "F.Cu") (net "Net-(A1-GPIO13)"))
 (segment (start 139.54 106) (end 137.62 104.08) (width 0.2) (layer "F.Cu") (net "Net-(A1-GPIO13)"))
 (segment (start 127.002292 82.795) (end 124.92 84.877292) (width 0.2) (layer "F.Cu") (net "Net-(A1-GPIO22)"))
 (segment (start 157.604744 82.795) (end 127.002292 82.795) (width 0.2) (layer "F.Cu") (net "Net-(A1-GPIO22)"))
 (segment (start 172.04 114.92) (end 172.04 97.230256) (width 0.2) (layer "F.Cu") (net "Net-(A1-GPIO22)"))
 (segment (start 124.92 84.877292) (end 124.92 85.5) (width 0.2) (layer "F.Cu") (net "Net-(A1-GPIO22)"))
 (segment (start 172.04 97.230256) (end 157.604744 82.795) (width 0.2) (layer "F.Cu") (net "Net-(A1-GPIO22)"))
 (segment (start 146.104364 114.92) (end 136.5 105.315636) (width 0.2) (layer "F.Cu") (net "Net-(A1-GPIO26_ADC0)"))
 (segment (start 136.5 99.411745) (end 126.988255 89.9) (width 0.2) (layer "F.Cu") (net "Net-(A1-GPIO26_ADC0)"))
 (segment (start 136.5 105.315636) (end 136.5 99.411745) (width 0.2) (layer "F.Cu") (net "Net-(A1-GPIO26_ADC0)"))
 (segment (start 126.988255 89.9) (end 124.24 89.9) (width 0.2) (layer "F.Cu") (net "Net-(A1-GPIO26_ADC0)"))
 (segment (start 150.54 114.92) (end 146.104364 114.92) (width 0.2) (layer "F.Cu") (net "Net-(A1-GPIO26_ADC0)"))
 (segment (start 124.24 89.9) (end 119.84 85.5) (width 0.2) (layer "F.Cu") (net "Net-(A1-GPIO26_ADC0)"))
 (segment (start 123.5 91.7) (end 117.3 85.5) (width 0.2) (layer "F.Cu") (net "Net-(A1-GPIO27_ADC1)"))
 (segment (start 129.04 115) (end 123.5 109.46) (width 0.2) (layer "F.Cu") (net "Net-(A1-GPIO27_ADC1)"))
 (segment (start 123.5 109.46) (end 123.5 91.7) (width 0.2) (layer "F.Cu") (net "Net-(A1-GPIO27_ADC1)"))
 (segment (start 113.4 86.68) (end 112.22 85.5) (width 0.2) (layer "F.Cu") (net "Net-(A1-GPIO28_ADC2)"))
 (segment (start 107.46 114.92) (end 113.4 108.98) (width 0.2) (layer "F.Cu") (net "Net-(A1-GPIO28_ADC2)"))
 (segment (start 113.4 108.98) (end 113.4 86.68) (width 0.2) (layer "F.Cu") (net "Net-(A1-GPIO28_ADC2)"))
 (segment (start 103.165 115.405) (end 103.165 99.535) (width 0.2) (layer "F.Cu") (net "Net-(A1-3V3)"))
 (segment (start 144.19 117.46) (end 122.77 117.46) (width 0.2) (layer "F.Cu") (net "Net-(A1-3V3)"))
 (segment (start 165.69 117.46) (end 144.19 117.46) (width 0.2) (layer "F.Cu") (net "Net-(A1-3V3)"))
 (segment (start 102.56 98.93) (end 102.56 90.08) (width 0.2) (layer "F.Cu") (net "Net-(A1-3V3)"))
 (segment (start 122.77 117.46) (end 122.69 117.54) (width 0.2) (layer "F.Cu") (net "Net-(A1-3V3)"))
 (segment (start 122.36 117.46) (end 101.11 117.46) (width 0.2) (layer "F.Cu") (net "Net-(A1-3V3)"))
 (segment (start 122.69 117.54) (end 122.44 117.54) (width 0.2) (layer "F.Cu") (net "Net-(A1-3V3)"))
 (segment (start 103.165 99.535) (end 102.56 98.93) (width 0.2) (layer "F.Cu") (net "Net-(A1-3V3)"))
 (segment (start 101.11 117.46) (end 103.165 115.405) (width 0.2) (layer "F.Cu") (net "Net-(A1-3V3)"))
 (segment (start 102.56 90.08) (end 107.14 85.5) (width 0.2) (layer "F.Cu") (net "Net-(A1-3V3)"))
 (segment (start 122.44 117.54) (end 122.36 117.46) (width 0.2) (layer "F.Cu") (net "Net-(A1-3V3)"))
 (segment (start 165.5 101) (end 165.5 95.9875) (width 0.2) (layer "F.Cu") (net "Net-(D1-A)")))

